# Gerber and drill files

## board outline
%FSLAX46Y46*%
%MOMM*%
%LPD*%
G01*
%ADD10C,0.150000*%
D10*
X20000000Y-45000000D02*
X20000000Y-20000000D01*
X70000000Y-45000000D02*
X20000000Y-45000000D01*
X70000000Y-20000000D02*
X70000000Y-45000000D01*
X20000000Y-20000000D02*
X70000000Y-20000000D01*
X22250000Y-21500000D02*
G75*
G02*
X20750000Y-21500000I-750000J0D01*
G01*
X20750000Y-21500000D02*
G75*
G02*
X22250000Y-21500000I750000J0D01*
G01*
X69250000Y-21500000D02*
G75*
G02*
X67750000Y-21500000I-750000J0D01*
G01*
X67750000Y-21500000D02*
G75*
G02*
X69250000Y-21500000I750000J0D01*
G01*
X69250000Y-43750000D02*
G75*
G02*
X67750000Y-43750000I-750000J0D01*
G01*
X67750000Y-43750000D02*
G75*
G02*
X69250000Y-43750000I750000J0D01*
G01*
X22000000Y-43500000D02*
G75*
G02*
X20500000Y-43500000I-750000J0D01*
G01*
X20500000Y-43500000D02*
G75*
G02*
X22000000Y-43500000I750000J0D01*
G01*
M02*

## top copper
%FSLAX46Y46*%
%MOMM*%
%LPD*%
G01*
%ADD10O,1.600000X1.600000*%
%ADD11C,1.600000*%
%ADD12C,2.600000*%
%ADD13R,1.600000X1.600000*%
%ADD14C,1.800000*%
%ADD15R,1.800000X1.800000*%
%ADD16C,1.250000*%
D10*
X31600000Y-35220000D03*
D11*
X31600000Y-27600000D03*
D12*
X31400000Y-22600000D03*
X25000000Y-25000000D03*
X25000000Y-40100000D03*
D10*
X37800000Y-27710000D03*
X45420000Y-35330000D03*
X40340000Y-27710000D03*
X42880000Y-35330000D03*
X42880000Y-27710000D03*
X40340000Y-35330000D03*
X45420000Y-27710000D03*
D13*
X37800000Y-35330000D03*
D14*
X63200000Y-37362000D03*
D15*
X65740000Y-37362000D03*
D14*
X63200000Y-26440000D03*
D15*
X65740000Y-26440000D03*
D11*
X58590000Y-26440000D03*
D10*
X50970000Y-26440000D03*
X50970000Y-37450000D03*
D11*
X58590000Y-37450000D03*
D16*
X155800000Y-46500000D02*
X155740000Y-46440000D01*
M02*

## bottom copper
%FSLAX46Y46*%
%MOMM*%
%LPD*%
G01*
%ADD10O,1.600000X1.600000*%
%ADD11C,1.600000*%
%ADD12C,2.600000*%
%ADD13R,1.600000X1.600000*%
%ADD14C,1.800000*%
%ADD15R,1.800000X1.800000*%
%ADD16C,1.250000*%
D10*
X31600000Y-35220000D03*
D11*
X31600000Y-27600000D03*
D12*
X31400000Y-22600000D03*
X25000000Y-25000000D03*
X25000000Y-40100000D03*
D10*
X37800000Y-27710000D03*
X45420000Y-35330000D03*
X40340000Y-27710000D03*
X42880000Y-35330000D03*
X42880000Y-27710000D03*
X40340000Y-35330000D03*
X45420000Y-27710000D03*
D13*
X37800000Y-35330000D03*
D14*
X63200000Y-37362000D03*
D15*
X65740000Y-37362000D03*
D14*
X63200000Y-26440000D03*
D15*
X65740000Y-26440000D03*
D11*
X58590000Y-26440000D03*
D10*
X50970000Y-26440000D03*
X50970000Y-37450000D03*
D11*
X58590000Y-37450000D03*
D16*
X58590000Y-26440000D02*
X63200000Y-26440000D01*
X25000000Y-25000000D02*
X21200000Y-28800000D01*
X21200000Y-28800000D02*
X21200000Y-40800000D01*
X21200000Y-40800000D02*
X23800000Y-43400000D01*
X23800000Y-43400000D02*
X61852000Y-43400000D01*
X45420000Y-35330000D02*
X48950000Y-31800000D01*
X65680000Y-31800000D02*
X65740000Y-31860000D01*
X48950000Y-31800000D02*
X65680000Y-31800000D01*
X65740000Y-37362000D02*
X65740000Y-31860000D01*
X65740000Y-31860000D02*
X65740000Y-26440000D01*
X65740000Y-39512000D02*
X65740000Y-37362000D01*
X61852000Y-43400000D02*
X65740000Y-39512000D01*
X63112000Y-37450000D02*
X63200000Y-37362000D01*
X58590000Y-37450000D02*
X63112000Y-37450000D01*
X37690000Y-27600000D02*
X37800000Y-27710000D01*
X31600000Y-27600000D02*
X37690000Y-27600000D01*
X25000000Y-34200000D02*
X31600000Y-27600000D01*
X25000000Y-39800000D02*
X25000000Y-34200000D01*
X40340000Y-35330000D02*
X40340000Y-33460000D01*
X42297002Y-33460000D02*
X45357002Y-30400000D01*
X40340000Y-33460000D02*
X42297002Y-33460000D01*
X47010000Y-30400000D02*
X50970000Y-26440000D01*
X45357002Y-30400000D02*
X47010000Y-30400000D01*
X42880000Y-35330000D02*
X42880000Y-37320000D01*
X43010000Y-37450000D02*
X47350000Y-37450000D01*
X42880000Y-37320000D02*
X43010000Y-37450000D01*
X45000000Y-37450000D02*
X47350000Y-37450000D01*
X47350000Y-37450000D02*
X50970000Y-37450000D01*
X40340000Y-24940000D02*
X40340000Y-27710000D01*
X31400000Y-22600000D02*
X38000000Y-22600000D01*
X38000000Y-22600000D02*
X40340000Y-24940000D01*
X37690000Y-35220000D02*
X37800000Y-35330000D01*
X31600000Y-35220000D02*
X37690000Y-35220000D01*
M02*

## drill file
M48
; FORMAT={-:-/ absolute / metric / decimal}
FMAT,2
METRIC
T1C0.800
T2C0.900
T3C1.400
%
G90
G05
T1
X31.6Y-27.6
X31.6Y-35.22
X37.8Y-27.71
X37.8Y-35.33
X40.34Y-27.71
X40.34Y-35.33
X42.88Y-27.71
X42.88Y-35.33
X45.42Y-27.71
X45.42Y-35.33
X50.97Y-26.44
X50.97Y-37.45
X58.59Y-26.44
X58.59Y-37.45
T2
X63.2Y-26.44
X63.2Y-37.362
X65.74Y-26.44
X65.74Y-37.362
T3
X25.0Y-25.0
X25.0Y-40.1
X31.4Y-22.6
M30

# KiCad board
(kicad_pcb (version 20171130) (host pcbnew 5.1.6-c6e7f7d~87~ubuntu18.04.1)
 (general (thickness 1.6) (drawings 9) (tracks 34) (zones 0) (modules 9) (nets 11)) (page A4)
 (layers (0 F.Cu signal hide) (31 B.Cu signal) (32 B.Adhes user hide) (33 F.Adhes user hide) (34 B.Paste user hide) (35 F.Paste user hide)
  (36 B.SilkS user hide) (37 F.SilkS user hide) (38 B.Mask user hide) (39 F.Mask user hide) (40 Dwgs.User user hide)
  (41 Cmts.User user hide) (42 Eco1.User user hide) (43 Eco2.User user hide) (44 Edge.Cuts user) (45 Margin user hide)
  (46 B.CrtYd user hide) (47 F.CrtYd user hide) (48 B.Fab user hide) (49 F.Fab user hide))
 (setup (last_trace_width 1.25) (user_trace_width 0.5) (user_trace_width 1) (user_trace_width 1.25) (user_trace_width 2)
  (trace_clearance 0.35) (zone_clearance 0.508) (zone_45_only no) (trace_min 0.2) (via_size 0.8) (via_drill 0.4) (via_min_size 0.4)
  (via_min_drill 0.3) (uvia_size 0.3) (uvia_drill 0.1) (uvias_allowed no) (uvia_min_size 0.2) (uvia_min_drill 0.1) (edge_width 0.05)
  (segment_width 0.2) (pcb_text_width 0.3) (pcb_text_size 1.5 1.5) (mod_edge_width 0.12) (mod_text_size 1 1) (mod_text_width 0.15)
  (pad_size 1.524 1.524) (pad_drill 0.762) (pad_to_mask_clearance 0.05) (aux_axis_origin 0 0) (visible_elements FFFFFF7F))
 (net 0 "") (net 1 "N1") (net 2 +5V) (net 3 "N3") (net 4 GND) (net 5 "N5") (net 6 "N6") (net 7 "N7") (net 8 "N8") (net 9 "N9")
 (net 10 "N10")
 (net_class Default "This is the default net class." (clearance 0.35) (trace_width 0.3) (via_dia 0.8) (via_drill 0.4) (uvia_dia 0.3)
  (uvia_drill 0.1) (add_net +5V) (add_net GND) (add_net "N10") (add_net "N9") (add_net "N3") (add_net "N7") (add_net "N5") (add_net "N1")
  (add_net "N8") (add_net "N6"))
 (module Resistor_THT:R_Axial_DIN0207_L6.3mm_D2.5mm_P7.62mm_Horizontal (layer F.Cu) (at 31.6 27.6 270)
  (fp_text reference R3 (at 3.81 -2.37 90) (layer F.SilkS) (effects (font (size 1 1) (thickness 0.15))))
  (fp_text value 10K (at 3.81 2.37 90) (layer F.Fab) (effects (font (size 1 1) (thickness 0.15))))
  (pad 2 thru_hole oval (at 7.62 0 270) (size 1.6 1.6) (drill 0.8) (layers *.Cu *.Mask) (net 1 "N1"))
  (pad 1 thru_hole circle (at 0 0 270) (size 1.6 1.6) (drill 0.8) (layers *.Cu *.Mask) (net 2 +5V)))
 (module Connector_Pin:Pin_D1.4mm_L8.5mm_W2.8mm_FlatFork (layer F.Cu) (at 31.4 22.6)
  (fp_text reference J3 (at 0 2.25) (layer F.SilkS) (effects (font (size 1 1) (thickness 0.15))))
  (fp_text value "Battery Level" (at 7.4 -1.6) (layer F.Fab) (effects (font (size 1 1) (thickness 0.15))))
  (pad 1 thru_hole circle (at 0 0) (size 2.6 2.6) (drill 1.4) (layers *.Cu *.Mask) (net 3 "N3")))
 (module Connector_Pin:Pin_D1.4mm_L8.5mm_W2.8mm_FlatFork (layer F.Cu) (at 25 25)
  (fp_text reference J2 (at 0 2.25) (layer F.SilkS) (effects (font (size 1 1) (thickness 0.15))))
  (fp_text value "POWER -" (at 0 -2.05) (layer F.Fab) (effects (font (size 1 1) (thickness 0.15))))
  (pad 1 thru_hole circle (at 0 0) (size 2.6 2.6) (drill 1.4) (layers *.Cu *.Mask) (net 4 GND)))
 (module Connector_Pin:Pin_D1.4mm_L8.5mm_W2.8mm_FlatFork (layer F.Cu) (at 25 40.1)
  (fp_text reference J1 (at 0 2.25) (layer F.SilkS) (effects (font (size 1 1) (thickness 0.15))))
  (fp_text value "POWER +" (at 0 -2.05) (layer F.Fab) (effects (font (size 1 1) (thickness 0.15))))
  (pad 1 thru_hole circle (at 0 0) (size 2.6 2.6) (drill 1.4) (layers *.Cu *.Mask) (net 2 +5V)))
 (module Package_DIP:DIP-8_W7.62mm (layer F.Cu) (at 37.8 35.33 90)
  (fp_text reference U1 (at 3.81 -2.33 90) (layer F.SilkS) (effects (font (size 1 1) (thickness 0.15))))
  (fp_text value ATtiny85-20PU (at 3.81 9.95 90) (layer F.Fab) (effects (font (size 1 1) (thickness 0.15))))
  (pad 8 thru_hole oval (at 7.62 0 90) (size 1.6 1.6) (drill 0.8) (layers *.Cu *.Mask) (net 2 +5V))
  (pad 4 thru_hole oval (at 0 7.62 90) (size 1.6 1.6) (drill 0.8) (layers *.Cu *.Mask) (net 4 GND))
  (pad 7 thru_hole oval (at 7.62 2.54 90) (size 1.6 1.6) (drill 0.8) (layers *.Cu *.Mask) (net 3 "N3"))
  (pad 3 thru_hole oval (at 0 5.08 90) (size 1.6 1.6) (drill 0.8) (layers *.Cu *.Mask) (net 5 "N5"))
  (pad 6 thru_hole oval (at 7.62 5.08 90) (size 1.6 1.6) (drill 0.8) (layers *.Cu *.Mask) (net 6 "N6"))
  (pad 2 thru_hole oval (at 0 2.54 90) (size 1.6 1.6) (drill 0.8) (layers *.Cu *.Mask) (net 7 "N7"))
  (pad 5 thru_hole oval (at 7.62 7.62 90) (size 1.6 1.6) (drill 0.8) (layers *.Cu *.Mask) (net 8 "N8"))
  (pad 1 thru_hole rect (at 0 0 90) (size 1.6 1.6) (drill 0.8) (layers *.Cu *.Mask) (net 1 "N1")))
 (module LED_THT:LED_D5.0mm (layer F.Cu) (at 65.74 37.362 180)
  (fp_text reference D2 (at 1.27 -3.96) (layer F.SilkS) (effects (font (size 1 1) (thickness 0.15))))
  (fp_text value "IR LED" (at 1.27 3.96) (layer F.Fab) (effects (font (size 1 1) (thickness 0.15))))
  (pad 2 thru_hole circle (at 2.54 0 180) (size 1.8 1.8) (drill 0.9) (layers *.Cu *.Mask) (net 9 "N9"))
  (pad 1 thru_hole rect (at 0 0 180) (size 1.8 1.8) (drill 0.9) (layers *.Cu *.Mask) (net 4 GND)))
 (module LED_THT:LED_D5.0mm (layer F.Cu) (at 65.74 26.44 180)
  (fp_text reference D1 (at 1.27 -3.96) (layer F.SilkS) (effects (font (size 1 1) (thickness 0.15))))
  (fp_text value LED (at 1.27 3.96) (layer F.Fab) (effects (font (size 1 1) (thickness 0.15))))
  (pad 2 thru_hole circle (at 2.54 0 180) (size 1.8 1.8) (drill 0.9) (layers *.Cu *.Mask) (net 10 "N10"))
  (pad 1 thru_hole rect (at 0 0 180) (size 1.8 1.8) (drill 0.9) (layers *.Cu *.Mask) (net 4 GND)))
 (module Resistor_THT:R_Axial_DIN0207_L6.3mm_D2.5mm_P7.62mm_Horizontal (layer F.Cu) (at 58.59 26.44 180)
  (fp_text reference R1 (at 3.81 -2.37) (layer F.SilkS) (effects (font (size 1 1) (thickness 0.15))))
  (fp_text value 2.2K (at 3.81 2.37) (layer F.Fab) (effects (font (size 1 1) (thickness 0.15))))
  (pad 1 thru_hole circle (at 0 0 180) (size 1.6 1.6) (drill 0.8) (layers *.Cu *.Mask) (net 10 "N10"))
  (pad 2 thru_hole oval (at 7.62 0 180) (size 1.6 1.6) (drill 0.8) (layers *.Cu *.Mask) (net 7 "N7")))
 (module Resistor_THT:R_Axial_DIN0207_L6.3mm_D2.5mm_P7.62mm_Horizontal (layer F.Cu) (at 58.59 37.45 180)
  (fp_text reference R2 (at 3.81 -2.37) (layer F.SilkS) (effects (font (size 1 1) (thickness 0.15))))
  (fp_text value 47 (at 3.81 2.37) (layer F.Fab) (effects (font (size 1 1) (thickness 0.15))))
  (pad 2 thru_hole oval (at 7.62 0 180) (size 1.6 1.6) (drill 0.8) (layers *.Cu *.Mask) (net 5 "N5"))
  (pad 1 thru_hole circle (at 0 0 180) (size 1.6 1.6) (drill 0.8) (layers *.Cu *.Mask) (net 9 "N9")))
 (gr_line (start 20 45) (end 20 20) (layer Edge.Cuts) (width 0.15))
 (gr_line (start 70 45) (end 20 45) (layer Edge.Cuts) (width 0.15))
 (gr_line (start 70 20) (end 70 45) (layer Edge.Cuts) (width 0.15))
 (gr_line (start 20 20) (end 70 20) (layer Edge.Cuts) (width 0.15))
 (gr_circle (center 21.5 21.5) (end 22.25 21.5) (layer Edge.Cuts) (width 0.15))
 (gr_circle (center 68.5 21.5) (end 69.25 21.5) (layer Edge.Cuts) (width 0.15))
 (gr_circle (center 68.5 43.75) (end 69.25 43.75) (layer Edge.Cuts) (width 0.15))
 (gr_circle (center 21.25 43.5) (end 22 43.5) (layer Edge.Cuts) (width 0.15))
 (segment (start 58.59 26.44) (end 63.2 26.44) (width 1.25) (layer B.Cu) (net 10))
 (segment (start 155.8 46.5) (end 155.74 46.44) (width 1.25) (layer F.Cu) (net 4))
 (segment (start 25 25) (end 21.2 28.8) (width 1.25) (layer B.Cu) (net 4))
 (segment (start 21.2 28.8) (end 21.2 40.8) (width 1.25) (layer B.Cu) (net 4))
 (segment (start 21.2 40.8) (end 23.8 43.4) (width 1.25) (layer B.Cu) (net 4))
 (segment (start 23.8 43.4) (end 61.852 43.4) (width 1.25) (layer B.Cu) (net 4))
 (segment (start 45.42 35.33) (end 48.95 31.8) (width 1.25) (layer B.Cu) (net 4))
 (segment (start 65.68 31.8) (end 65.74 31.86) (width 1.25) (layer B.Cu) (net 4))
 (segment (start 48.95 31.8) (end 65.68 31.8) (width 1.25) (layer B.Cu) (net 4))
 (segment (start 65.74 37.362) (end 65.74 31.86) (width 1.25) (layer B.Cu) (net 4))
 (segment (start 65.74 31.86) (end 65.74 26.44) (width 1.25) (layer B.Cu) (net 4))
 (segment (start 65.74 39.512) (end 65.74 37.362) (width 1.25) (layer B.Cu) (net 4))
 (segment (start 61.852 43.4) (end 65.74 39.512) (width 1.25) (layer B.Cu) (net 4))
 (segment (start 63.112 37.45) (end 63.2 37.362) (width 1.25) (layer B.Cu) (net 9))
 (segment (start 58.59 37.45) (end 63.112 37.45) (width 1.25) (layer B.Cu) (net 9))
 (segment (start 37.69 27.6) (end 37.8 27.71) (width 1.25) (layer B.Cu) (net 2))
 (segment (start 31.6 27.6) (end 37.69 27.6) (width 1.25) (layer B.Cu) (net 2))
 (segment (start 25 34.2) (end 31.6 27.6) (width 1.25) (layer B.Cu) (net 2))
 (segment (start 25 39.8) (end 25 34.2) (width 1.25) (layer B.Cu) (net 2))
 (segment (start 40.34 35.33) (end 40.34 33.46) (width 1.25) (layer B.Cu) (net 7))
 (segment (start 42.297002 33.46) (end 45.357002 30.4) (width 1.25) (layer B.Cu) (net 7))
 (segment (start 40.34 33.46) (end 42.297002 33.46) (width 1.25) (layer B.Cu) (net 7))
 (segment (start 47.01 30.4) (end 50.97 26.44) (width 1.25) (layer B.Cu) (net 7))
 (segment (start 45.357002 30.4) (end 47.01 30.4) (width 1.25) (layer B.Cu) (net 7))
 (segment (start 42.88 35.33) (end 42.88 37.32) (width 1.25) (layer B.Cu) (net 5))
 (segment (start 43.01 37.45) (end 47.35 37.45) (width 1.25) (layer B.Cu) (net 5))
 (segment (start 42.88 37.32) (end 43.01 37.45) (width 1.25) (layer B.Cu) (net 5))
 (segment (start 45 37.45) (end 47.35 37.45) (width 1.25) (layer B.Cu) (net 5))
 (segment (start 47.35 37.45) (end 50.97 37.45) (width 1.25) (layer B.Cu) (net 5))
 (segment (start 40.34 24.94) (end 40.34 27.71) (width 1.25) (layer B.Cu) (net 3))
 (segment (start 31.4 22.6) (end 38 22.6) (width 1.25) (layer B.Cu) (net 3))
 (segment (start 38 22.6) (end 40.34 24.94) (width 1.25) (layer B.Cu) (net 3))
 (segment (start 37.69 35.22) (end 37.8 35.33) (width 1.25) (layer B.Cu) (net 1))
 (segment (start 31.6 35.22) (end 37.69 35.22) (width 1.25) (layer B.Cu) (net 1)))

